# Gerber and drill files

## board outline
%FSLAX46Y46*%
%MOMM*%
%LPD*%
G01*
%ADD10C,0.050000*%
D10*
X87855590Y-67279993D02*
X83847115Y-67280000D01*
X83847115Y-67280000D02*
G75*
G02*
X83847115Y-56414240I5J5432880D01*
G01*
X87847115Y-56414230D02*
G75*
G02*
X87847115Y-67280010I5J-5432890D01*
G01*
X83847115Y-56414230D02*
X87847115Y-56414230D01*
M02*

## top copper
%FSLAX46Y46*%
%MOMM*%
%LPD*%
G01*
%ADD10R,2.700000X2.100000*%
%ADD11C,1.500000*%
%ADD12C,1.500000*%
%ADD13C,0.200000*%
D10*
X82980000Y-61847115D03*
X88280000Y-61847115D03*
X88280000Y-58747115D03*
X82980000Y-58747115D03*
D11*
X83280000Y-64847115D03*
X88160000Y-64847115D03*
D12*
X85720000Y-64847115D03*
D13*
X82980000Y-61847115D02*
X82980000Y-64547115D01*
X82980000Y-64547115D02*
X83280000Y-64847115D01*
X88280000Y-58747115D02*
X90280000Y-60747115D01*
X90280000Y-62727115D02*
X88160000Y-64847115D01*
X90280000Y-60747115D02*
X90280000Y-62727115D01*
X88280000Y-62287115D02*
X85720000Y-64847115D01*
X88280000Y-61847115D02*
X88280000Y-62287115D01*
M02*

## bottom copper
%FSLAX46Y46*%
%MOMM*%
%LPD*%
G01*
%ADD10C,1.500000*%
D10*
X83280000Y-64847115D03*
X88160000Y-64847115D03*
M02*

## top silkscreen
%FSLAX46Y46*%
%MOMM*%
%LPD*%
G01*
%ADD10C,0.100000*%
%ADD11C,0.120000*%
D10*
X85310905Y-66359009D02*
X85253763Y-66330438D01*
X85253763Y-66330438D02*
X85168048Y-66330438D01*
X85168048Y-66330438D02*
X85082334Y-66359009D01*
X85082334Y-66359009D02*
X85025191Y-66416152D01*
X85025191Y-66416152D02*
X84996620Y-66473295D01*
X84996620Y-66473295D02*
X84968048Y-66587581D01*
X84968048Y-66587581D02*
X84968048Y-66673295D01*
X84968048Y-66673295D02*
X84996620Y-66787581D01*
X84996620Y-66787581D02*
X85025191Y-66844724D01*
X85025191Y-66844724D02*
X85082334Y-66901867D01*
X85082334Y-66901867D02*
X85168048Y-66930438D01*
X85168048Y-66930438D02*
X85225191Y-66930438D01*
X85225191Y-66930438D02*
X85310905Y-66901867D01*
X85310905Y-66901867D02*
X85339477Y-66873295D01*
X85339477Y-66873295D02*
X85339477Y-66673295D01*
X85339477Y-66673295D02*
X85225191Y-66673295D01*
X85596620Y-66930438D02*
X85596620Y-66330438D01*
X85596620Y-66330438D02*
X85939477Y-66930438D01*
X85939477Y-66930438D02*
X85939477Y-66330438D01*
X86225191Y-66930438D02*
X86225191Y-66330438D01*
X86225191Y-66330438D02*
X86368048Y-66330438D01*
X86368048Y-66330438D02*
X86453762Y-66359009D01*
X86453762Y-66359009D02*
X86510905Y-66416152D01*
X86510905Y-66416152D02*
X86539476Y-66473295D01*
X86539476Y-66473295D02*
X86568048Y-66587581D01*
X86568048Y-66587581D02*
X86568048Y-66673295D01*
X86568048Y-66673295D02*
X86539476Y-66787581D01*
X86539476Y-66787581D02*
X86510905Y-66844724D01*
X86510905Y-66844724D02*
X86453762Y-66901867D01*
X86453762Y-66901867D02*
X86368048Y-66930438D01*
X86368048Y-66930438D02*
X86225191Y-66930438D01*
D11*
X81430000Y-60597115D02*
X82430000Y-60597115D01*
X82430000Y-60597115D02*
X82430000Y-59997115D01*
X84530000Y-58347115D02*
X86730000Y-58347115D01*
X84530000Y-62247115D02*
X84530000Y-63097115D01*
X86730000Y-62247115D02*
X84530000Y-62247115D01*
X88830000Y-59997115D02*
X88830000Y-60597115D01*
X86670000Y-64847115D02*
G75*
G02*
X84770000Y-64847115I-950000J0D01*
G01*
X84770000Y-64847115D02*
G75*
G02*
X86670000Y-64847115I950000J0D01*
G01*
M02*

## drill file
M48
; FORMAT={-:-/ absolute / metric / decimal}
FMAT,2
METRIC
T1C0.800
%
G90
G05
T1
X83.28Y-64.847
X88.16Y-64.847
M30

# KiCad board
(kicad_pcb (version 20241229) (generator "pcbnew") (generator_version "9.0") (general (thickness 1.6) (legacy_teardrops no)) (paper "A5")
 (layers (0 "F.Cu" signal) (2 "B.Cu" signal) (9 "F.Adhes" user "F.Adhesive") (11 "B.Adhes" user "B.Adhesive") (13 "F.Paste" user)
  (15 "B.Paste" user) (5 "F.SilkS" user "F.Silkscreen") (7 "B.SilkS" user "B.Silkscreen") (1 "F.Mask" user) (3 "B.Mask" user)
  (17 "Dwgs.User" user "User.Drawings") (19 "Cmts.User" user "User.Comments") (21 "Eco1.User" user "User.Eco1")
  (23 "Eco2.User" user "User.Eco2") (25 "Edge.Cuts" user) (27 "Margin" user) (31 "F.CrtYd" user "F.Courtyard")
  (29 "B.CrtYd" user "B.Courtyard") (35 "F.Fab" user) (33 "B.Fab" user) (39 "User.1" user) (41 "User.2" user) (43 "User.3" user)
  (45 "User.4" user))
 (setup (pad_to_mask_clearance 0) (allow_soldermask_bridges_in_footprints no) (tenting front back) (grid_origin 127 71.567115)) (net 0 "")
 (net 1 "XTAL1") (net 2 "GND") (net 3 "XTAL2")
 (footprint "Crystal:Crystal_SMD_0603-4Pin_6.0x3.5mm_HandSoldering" (layer "F.Cu") (at 85.63 60.297115)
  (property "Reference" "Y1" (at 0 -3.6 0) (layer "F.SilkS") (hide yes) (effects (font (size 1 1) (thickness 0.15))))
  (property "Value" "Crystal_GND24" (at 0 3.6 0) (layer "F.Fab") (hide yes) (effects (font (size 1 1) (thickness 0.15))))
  (fp_line (start -4.2 0.3) (end -3.2 0.3) (stroke (width 0.12) (type solid)) (layer "F.SilkS"))
  (fp_line (start -3.2 0.3) (end -3.2 -0.3) (stroke (width 0.12) (type solid)) (layer "F.SilkS"))
  (fp_line (start -1.1 -1.95) (end 1.1 -1.95) (stroke (width 0.12) (type solid)) (layer "F.SilkS"))
  (fp_line (start -1.1 1.95) (end -1.1 2.8) (stroke (width 0.12) (type solid)) (layer "F.SilkS"))
  (fp_line (start 1.1 1.95) (end -1.1 1.95) (stroke (width 0.12) (type solid)) (layer "F.SilkS"))
  (fp_line (start 3.2 -0.3) (end 3.2 0.3) (stroke (width 0.12) (type solid)) (layer "F.SilkS"))
  (pad "1" smd rect (at -2.65 1.55) (size 2.7 2.1) (layers "F.Cu" "F.Mask" "F.Paste") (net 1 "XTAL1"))
  (pad "2" smd rect (at 2.65 1.55) (size 2.7 2.1) (layers "F.Cu" "F.Mask" "F.Paste") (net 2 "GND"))
  (pad "3" smd rect (at 2.65 -1.55) (size 2.7 2.1) (layers "F.Cu" "F.Mask" "F.Paste") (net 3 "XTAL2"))
  (pad "4" smd rect (at -2.65 -1.55) (size 2.7 2.1) (layers "F.Cu" "F.Mask" "F.Paste") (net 2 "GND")))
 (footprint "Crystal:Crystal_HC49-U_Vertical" (layer "F.Cu") (at 83.28 64.847115)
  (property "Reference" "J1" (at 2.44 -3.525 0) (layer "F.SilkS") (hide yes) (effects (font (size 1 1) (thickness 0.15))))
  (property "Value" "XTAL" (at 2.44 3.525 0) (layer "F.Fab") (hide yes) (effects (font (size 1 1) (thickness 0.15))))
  (pad "1" thru_hole circle (at 0 0) (size 1.5 1.5) (drill 0.8) (layers "*.Cu" "*.Mask") (remove_unused_layers no) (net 1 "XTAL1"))
  (pad "2" thru_hole circle (at 4.88 0) (size 1.5 1.5) (drill 0.8) (layers "*.Cu" "*.Mask") (remove_unused_layers no) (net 3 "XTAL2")))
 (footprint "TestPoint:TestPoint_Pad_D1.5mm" (layer "F.Cu") (at 85.72 64.847115)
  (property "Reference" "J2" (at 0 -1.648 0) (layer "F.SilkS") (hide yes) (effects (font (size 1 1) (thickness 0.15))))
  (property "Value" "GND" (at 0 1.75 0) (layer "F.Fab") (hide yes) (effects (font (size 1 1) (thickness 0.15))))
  (fp_circle (center 0 0) (end 0 0.95) (stroke (width 0.12) (type solid)) (fill no) (layer "F.SilkS"))
  (pad "1" smd circle (at 0 0) (size 1.5 1.5) (layers "F.Cu" "F.Mask") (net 2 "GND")))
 (gr_line (start 87.85559 67.279993) (end 83.847115 67.28) (stroke (width 0.05) (type default)) (layer "Edge.Cuts"))
 (gr_arc (start 83.847115 67.28) (mid 78.41423 61.847115) (end 83.847115 56.41423) (stroke (width 0.05) (type default)) (layer "Edge.Cuts"))
 (gr_arc (start 87.847115 56.41423) (mid 93.28 61.847115) (end 87.847115 67.28) (stroke (width 0.05) (type default)) (layer "Edge.Cuts"))
 (gr_line (start 83.847115 56.41423) (end 87.847115 56.41423) (stroke (width 0.05) (type default)) (layer "Edge.Cuts"))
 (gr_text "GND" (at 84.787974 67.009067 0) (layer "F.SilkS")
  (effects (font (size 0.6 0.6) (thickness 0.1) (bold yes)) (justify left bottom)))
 (segment (start 82.98 61.847115) (end 82.98 64.547115) (width 0.2) (layer "F.Cu") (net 1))
 (segment (start 82.98 64.547115) (end 83.28 64.847115) (width 0.2) (layer "F.Cu") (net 1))
 (segment (start 88.28 58.747115) (end 90.28 60.747115) (width 0.2) (layer "F.Cu") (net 3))
 (segment (start 90.28 62.727115) (end 88.16 64.847115) (width 0.2) (layer "F.Cu") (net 3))
 (segment (start 90.28 60.747115) (end 90.28 62.727115) (width 0.2) (layer "F.Cu") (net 3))
 (segment (start 88.28 62.287115) (end 85.72 64.847115) (width 0.2) (layer "F.Cu") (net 2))
 (segment (start 88.28 61.847115) (end 88.28 62.287115) (width 0.2) (layer "F.Cu") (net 2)))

